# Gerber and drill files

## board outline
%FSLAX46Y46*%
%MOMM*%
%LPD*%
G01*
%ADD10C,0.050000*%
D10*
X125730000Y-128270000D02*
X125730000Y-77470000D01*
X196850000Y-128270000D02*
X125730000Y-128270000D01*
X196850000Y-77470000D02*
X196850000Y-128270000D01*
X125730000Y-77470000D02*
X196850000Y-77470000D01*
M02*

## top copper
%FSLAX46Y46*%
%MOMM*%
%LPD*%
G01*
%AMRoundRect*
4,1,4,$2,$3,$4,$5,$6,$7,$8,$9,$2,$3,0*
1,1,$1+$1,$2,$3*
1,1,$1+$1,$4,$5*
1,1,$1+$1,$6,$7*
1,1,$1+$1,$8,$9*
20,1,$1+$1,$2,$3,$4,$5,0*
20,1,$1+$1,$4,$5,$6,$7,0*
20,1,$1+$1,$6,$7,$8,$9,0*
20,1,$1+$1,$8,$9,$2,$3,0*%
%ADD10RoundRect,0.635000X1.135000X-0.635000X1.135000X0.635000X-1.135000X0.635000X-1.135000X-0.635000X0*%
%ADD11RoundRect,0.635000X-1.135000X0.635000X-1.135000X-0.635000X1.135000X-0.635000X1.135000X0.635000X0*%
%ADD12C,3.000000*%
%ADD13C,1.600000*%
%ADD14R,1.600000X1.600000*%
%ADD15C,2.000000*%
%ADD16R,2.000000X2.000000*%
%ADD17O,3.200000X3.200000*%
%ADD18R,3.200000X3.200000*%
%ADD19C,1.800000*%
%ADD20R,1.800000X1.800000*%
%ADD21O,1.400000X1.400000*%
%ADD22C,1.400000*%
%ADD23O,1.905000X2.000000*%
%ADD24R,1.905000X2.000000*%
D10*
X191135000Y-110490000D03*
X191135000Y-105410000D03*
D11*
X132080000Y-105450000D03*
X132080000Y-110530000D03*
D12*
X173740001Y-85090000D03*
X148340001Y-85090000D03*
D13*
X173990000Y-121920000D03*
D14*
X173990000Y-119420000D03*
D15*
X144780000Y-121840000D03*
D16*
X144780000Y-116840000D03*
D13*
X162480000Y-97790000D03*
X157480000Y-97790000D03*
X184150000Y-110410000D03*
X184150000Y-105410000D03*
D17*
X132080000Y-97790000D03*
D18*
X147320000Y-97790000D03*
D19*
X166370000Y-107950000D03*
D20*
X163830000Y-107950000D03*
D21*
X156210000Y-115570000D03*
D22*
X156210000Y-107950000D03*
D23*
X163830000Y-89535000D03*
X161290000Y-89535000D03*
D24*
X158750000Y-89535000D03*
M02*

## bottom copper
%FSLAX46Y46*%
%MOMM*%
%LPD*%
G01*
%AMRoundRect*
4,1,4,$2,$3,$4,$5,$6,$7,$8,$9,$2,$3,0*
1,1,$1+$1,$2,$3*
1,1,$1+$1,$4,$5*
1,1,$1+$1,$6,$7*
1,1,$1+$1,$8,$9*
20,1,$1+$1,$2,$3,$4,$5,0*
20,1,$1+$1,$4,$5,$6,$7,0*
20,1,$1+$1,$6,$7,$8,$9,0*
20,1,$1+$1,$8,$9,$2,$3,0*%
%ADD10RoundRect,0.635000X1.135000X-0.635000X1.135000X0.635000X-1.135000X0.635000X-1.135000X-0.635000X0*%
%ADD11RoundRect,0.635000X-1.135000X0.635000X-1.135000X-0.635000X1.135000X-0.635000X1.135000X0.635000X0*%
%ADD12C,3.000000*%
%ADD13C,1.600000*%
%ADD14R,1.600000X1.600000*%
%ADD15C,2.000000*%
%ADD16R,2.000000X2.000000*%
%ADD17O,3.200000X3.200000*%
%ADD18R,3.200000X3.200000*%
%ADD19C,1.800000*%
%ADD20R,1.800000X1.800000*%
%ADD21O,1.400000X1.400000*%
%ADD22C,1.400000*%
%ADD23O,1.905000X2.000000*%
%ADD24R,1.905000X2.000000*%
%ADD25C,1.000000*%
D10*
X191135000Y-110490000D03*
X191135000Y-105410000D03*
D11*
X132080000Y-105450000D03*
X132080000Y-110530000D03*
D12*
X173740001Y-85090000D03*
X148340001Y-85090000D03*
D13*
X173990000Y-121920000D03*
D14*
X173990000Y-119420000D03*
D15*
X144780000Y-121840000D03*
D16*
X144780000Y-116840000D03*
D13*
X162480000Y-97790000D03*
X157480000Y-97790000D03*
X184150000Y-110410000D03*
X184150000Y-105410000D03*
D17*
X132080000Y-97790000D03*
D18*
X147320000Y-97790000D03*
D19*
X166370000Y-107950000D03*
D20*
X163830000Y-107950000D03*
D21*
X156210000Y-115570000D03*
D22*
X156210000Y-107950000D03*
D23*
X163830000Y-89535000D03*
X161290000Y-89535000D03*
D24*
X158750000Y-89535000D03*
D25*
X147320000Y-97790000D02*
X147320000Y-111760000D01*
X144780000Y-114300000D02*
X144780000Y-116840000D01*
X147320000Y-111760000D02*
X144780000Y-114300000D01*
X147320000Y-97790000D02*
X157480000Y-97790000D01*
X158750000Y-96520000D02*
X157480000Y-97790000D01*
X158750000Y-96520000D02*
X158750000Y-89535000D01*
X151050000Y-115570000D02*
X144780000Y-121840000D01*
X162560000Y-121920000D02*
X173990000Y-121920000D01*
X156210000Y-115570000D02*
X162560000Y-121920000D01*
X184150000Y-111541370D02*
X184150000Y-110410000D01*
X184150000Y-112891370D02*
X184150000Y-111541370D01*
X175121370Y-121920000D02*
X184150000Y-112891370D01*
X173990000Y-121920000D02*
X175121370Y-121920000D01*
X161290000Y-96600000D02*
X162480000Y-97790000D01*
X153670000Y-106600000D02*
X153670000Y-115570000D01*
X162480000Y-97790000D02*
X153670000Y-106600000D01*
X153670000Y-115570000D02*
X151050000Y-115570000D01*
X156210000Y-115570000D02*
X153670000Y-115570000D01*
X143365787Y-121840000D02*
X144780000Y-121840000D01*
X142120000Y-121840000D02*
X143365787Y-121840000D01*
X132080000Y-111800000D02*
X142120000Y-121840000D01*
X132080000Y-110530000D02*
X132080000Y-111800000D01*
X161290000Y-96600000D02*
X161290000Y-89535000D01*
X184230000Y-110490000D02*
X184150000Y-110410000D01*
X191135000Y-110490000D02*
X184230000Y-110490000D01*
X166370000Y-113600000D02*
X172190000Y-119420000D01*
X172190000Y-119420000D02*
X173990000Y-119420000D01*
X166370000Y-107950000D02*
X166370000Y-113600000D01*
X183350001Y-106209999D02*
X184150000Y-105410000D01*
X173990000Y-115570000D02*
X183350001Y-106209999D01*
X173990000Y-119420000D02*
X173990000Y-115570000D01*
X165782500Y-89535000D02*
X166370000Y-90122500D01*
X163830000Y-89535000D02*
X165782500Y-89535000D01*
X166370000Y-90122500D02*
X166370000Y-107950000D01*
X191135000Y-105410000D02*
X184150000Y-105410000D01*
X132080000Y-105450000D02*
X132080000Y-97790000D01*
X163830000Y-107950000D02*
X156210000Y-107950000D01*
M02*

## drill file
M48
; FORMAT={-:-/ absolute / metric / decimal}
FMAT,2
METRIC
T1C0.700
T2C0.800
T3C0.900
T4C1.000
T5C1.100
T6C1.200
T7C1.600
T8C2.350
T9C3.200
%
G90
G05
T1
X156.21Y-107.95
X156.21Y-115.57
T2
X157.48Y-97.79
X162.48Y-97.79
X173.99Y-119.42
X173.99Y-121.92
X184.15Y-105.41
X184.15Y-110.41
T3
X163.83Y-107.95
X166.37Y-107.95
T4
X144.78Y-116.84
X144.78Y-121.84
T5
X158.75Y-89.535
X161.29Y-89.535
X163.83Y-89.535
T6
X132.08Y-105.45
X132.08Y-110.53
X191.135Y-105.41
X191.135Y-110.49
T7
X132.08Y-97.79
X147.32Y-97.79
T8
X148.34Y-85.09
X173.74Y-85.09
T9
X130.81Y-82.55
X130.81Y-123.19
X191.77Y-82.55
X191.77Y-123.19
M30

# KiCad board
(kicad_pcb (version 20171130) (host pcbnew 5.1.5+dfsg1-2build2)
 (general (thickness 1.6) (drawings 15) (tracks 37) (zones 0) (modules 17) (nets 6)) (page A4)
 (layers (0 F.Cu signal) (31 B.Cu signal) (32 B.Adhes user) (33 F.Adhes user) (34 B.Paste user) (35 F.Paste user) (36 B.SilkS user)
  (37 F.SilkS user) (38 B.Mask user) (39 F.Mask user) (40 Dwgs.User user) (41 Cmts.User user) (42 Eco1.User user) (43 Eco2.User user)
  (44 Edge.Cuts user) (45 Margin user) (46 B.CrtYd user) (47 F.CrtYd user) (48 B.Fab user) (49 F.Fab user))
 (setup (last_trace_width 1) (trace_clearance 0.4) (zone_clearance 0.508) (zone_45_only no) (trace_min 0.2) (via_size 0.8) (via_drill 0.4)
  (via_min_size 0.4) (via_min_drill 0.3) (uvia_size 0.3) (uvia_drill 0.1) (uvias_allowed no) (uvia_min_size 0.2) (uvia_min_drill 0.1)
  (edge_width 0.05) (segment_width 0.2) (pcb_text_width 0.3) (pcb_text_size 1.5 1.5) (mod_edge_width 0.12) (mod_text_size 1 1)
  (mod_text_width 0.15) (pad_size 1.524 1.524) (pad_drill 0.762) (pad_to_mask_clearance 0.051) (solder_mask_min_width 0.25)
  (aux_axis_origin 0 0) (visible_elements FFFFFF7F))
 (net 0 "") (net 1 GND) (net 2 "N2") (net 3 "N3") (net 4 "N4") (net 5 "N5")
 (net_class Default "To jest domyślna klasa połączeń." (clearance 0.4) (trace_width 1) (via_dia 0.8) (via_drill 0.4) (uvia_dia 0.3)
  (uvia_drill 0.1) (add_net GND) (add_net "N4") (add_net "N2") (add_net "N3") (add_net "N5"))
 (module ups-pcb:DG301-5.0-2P (layer F.Cu) (at 191.135 107.99 90)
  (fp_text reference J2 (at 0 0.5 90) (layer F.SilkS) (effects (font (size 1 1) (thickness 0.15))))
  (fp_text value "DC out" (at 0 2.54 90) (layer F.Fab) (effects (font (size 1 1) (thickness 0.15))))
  (pad 1 thru_hole roundrect (at -2.5 0 90) (size 2.54 3.54) (drill 1.2) (layers *.Cu *.Mask) (roundrect_rratio 0.25) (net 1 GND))
  (pad 2 thru_hole roundrect (at 2.58 0 90) (size 2.54 3.54) (drill 1.2) (layers *.Cu *.Mask) (roundrect_rratio 0.25) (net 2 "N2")))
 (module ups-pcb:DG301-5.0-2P (layer F.Cu) (at 132.08 107.95 270)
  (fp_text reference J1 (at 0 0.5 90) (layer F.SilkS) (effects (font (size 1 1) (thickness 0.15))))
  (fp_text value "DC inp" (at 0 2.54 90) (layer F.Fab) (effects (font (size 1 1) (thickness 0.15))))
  (pad 1 thru_hole roundrect (at -2.5 0 270) (size 2.54 3.54) (drill 1.2) (layers *.Cu *.Mask) (roundrect_rratio 0.25) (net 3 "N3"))
  (pad 2 thru_hole roundrect (at 2.58 0 270) (size 2.54 3.54) (drill 1.2) (layers *.Cu *.Mask) (roundrect_rratio 0.25) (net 1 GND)))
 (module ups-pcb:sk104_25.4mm (layer F.Cu) (at 161.040001 85.09)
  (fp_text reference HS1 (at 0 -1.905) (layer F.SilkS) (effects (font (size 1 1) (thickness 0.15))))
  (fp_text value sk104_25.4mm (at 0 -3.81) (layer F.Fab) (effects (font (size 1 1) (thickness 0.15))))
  (pad "" np_thru_hole circle (at 12.7 0) (size 3 3) (drill 2.35) (layers *.Cu *.Mask))
  (pad "" np_thru_hole circle (at -12.7 0) (size 3 3) (drill 2.35) (layers *.Cu *.Mask)))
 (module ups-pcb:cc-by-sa (layer F.Cu) (at 159.385 121.92)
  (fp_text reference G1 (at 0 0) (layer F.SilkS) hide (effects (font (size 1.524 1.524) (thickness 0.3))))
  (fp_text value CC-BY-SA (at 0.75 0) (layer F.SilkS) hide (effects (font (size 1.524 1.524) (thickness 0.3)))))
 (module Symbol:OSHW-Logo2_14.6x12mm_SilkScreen (layer F.Cu) (at 186.055 93.98)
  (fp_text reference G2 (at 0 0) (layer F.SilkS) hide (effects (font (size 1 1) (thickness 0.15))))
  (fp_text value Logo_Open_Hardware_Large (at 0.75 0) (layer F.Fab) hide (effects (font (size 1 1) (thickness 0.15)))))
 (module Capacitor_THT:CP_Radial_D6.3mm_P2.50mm (layer F.Cu) (at 173.99 119.42 270)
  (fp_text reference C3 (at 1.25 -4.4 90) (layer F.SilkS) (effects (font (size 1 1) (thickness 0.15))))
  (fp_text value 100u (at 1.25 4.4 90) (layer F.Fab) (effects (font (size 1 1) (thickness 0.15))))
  (pad 2 thru_hole circle (at 2.5 0 270) (size 1.6 1.6) (drill 0.8) (layers *.Cu *.Mask) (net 1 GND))
  (pad 1 thru_hole rect (at 0 0 270) (size 1.6 1.6) (drill 0.8) (layers *.Cu *.Mask) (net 2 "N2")))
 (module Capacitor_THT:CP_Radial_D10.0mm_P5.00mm (layer F.Cu) (at 144.78 116.84 270)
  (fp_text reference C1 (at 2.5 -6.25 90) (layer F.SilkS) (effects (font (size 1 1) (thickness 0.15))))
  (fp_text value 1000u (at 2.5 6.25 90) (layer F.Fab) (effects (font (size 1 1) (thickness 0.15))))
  (pad 2 thru_hole circle (at 5 0 270) (size 2 2) (drill 1) (layers *.Cu *.Mask) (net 1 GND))
  (pad 1 thru_hole rect (at 0 0 270) (size 2 2) (drill 1) (layers *.Cu *.Mask) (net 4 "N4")))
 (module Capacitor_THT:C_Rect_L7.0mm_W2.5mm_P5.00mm (layer F.Cu) (at 157.48 97.79)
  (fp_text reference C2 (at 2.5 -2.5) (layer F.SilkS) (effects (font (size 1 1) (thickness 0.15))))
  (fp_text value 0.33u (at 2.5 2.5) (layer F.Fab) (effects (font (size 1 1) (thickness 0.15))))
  (pad 2 thru_hole circle (at 5 0) (size 1.6 1.6) (drill 0.8) (layers *.Cu *.Mask) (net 1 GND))
  (pad 1 thru_hole circle (at 0 0) (size 1.6 1.6) (drill 0.8) (layers *.Cu *.Mask) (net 4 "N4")))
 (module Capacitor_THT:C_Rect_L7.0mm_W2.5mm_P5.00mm (layer F.Cu) (at 184.15 105.41 270)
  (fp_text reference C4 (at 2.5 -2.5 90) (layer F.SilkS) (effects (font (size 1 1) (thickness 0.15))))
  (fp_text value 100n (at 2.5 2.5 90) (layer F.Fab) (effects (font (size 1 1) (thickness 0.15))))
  (pad 2 thru_hole circle (at 5 0 270) (size 1.6 1.6) (drill 0.8) (layers *.Cu *.Mask) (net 1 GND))
  (pad 1 thru_hole circle (at 0 0 270) (size 1.6 1.6) (drill 0.8) (layers *.Cu *.Mask) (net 2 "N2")))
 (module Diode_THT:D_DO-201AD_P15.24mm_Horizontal (layer F.Cu) (at 147.32 97.79 180)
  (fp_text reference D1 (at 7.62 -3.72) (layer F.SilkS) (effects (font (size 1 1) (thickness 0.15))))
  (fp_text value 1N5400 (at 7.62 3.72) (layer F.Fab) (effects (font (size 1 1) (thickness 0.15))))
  (pad 2 thru_hole oval (at 15.24 0 180) (size 3.2 3.2) (drill 1.6) (layers *.Cu *.Mask) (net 3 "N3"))
  (pad 1 thru_hole rect (at 0 0 180) (size 3.2 3.2) (drill 1.6) (layers *.Cu *.Mask) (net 4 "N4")))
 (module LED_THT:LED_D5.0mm (layer F.Cu) (at 163.83 107.95)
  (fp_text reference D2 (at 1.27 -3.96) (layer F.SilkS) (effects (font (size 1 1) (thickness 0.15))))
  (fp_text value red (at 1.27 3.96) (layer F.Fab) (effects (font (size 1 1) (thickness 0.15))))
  (pad 2 thru_hole circle (at 2.54 0) (size 1.8 1.8) (drill 0.9) (layers *.Cu *.Mask) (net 2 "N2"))
  (pad 1 thru_hole rect (at 0 0) (size 1.8 1.8) (drill 0.9) (layers *.Cu *.Mask) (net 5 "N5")))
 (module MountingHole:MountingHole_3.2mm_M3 (layer F.Cu) (at 130.81 82.55)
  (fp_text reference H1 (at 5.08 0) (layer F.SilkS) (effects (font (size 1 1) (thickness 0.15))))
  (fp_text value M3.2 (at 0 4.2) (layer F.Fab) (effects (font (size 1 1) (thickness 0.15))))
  (pad 1 np_thru_hole circle (at 0 0) (size 3.2 3.2) (drill 3.2) (layers *.Cu *.Mask)))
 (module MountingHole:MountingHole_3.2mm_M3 (layer F.Cu) (at 191.77 82.55)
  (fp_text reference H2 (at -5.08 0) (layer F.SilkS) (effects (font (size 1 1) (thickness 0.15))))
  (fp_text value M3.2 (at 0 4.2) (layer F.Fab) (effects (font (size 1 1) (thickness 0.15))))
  (pad 1 np_thru_hole circle (at 0 0) (size 3.2 3.2) (drill 3.2) (layers *.Cu *.Mask)))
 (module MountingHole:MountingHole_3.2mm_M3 (layer F.Cu) (at 191.77 123.19)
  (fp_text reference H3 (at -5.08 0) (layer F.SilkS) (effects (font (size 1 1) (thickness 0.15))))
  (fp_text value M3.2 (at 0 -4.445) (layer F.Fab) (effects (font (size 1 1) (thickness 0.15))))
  (pad 1 np_thru_hole circle (at 0 0) (size 3.2 3.2) (drill 3.2) (layers *.Cu *.Mask)))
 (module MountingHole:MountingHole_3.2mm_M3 (layer F.Cu) (at 130.81 123.19)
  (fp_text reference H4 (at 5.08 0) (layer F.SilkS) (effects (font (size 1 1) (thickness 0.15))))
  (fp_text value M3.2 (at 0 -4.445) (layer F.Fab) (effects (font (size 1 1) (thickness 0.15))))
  (pad 1 np_thru_hole circle (at 0 0) (size 3.2 3.2) (drill 3.2) (layers *.Cu *.Mask)))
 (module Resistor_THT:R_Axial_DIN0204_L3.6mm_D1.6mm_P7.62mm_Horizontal (layer F.Cu) (at 156.21 107.95 270)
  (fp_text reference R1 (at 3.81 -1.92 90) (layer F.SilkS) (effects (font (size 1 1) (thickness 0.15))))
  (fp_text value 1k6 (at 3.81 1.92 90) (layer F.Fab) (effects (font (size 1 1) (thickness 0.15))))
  (pad 2 thru_hole oval (at 7.62 0 270) (size 1.4 1.4) (drill 0.7) (layers *.Cu *.Mask) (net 1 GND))
  (pad 1 thru_hole circle (at 0 0 270) (size 1.4 1.4) (drill 0.7) (layers *.Cu *.Mask) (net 5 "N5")))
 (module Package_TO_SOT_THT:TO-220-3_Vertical (layer F.Cu) (at 158.75 89.535)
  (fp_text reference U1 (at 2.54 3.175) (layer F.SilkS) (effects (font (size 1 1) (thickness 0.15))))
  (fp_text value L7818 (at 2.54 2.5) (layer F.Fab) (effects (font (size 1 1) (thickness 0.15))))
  (pad 3 thru_hole oval (at 5.08 0) (size 1.905 2) (drill 1.1) (layers *.Cu *.Mask) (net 2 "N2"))
  (pad 2 thru_hole oval (at 2.54 0) (size 1.905 2) (drill 1.1) (layers *.Cu *.Mask) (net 1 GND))
  (pad 1 thru_hole rect (at 0 0) (size 1.905 2) (drill 1.1) (layers *.Cu *.Mask) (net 4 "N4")))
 (gr_line (start 125.73 128.27) (end 125.73 77.47) (layer Edge.Cuts) (width 0.05))
 (gr_line (start 196.85 128.27) (end 125.73 128.27) (layer Edge.Cuts) (width 0.05))
 (gr_line (start 196.85 77.47) (end 196.85 128.27) (layer Edge.Cuts) (width 0.05))
 (gr_line (start 125.73 77.47) (end 196.85 77.47) (layer Edge.Cuts) (width 0.05))
 (segment (start 147.32 97.79) (end 147.32 111.76) (width 1) (layer B.Cu) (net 4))
 (segment (start 144.78 114.3) (end 144.78 116.84) (width 1) (layer B.Cu) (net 4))
 (segment (start 147.32 111.76) (end 144.78 114.3) (width 1) (layer B.Cu) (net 4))
 (segment (start 147.32 97.79) (end 157.48 97.79) (width 1) (layer B.Cu) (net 4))
 (segment (start 158.75 96.52) (end 157.48 97.79) (width 1) (layer B.Cu) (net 4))
 (segment (start 158.75 96.52) (end 158.75 89.535) (width 1) (layer B.Cu) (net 4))
 (segment (start 151.05 115.57) (end 144.78 121.84) (width 1) (layer B.Cu) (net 1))
 (segment (start 162.56 121.92) (end 173.99 121.92) (width 1) (layer B.Cu) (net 1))
 (segment (start 156.21 115.57) (end 162.56 121.92) (width 1) (layer B.Cu) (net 1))
 (segment (start 184.15 111.54137) (end 184.15 110.41) (width 1) (layer B.Cu) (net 1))
 (segment (start 184.15 112.89137) (end 184.15 111.54137) (width 1) (layer B.Cu) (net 1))
 (segment (start 175.12137 121.92) (end 184.15 112.89137) (width 1) (layer B.Cu) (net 1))
 (segment (start 173.99 121.92) (end 175.12137 121.92) (width 1) (layer B.Cu) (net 1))
 (segment (start 161.29 96.6) (end 162.48 97.79) (width 1) (layer B.Cu) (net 1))
 (segment (start 153.67 106.6) (end 153.67 115.57) (width 1) (layer B.Cu) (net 1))
 (segment (start 162.48 97.79) (end 153.67 106.6) (width 1) (layer B.Cu) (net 1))
 (segment (start 153.67 115.57) (end 151.05 115.57) (width 1) (layer B.Cu) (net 1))
 (segment (start 156.21 115.57) (end 153.67 115.57) (width 1) (layer B.Cu) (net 1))
 (segment (start 143.365787 121.84) (end 144.78 121.84) (width 1) (layer B.Cu) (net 1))
 (segment (start 142.12 121.84) (end 143.365787 121.84) (width 1) (layer B.Cu) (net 1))
 (segment (start 132.08 111.8) (end 142.12 121.84) (width 1) (layer B.Cu) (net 1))
 (segment (start 132.08 110.53) (end 132.08 111.8) (width 1) (layer B.Cu) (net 1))
 (segment (start 161.29 96.6) (end 161.29 89.535) (width 1) (layer B.Cu) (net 1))
 (segment (start 184.23 110.49) (end 184.15 110.41) (width 1) (layer B.Cu) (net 1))
 (segment (start 191.135 110.49) (end 184.23 110.49) (width 1) (layer B.Cu) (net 1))
 (segment (start 166.37 113.6) (end 172.19 119.42) (width 1) (layer B.Cu) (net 2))
 (segment (start 172.19 119.42) (end 173.99 119.42) (width 1) (layer B.Cu) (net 2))
 (segment (start 166.37 107.95) (end 166.37 113.6) (width 1) (layer B.Cu) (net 2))
 (segment (start 183.350001 106.209999) (end 184.15 105.41) (width 1) (layer B.Cu) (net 2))
 (segment (start 173.99 115.57) (end 183.350001 106.209999) (width 1) (layer B.Cu) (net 2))
 (segment (start 173.99 119.42) (end 173.99 115.57) (width 1) (layer B.Cu) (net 2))
 (segment (start 165.7825 89.535) (end 166.37 90.1225) (width 1) (layer B.Cu) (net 2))
 (segment (start 163.83 89.535) (end 165.7825 89.535) (width 1) (layer B.Cu) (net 2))
 (segment (start 166.37 90.1225) (end 166.37 107.95) (width 1) (layer B.Cu) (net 2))
 (segment (start 191.135 105.41) (end 184.15 105.41) (width 1) (layer B.Cu) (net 2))
 (segment (start 132.08 105.45) (end 132.08 97.79) (width 1) (layer B.Cu) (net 3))
 (segment (start 163.83 107.95) (end 156.21 107.95) (width 1) (layer B.Cu) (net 5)))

